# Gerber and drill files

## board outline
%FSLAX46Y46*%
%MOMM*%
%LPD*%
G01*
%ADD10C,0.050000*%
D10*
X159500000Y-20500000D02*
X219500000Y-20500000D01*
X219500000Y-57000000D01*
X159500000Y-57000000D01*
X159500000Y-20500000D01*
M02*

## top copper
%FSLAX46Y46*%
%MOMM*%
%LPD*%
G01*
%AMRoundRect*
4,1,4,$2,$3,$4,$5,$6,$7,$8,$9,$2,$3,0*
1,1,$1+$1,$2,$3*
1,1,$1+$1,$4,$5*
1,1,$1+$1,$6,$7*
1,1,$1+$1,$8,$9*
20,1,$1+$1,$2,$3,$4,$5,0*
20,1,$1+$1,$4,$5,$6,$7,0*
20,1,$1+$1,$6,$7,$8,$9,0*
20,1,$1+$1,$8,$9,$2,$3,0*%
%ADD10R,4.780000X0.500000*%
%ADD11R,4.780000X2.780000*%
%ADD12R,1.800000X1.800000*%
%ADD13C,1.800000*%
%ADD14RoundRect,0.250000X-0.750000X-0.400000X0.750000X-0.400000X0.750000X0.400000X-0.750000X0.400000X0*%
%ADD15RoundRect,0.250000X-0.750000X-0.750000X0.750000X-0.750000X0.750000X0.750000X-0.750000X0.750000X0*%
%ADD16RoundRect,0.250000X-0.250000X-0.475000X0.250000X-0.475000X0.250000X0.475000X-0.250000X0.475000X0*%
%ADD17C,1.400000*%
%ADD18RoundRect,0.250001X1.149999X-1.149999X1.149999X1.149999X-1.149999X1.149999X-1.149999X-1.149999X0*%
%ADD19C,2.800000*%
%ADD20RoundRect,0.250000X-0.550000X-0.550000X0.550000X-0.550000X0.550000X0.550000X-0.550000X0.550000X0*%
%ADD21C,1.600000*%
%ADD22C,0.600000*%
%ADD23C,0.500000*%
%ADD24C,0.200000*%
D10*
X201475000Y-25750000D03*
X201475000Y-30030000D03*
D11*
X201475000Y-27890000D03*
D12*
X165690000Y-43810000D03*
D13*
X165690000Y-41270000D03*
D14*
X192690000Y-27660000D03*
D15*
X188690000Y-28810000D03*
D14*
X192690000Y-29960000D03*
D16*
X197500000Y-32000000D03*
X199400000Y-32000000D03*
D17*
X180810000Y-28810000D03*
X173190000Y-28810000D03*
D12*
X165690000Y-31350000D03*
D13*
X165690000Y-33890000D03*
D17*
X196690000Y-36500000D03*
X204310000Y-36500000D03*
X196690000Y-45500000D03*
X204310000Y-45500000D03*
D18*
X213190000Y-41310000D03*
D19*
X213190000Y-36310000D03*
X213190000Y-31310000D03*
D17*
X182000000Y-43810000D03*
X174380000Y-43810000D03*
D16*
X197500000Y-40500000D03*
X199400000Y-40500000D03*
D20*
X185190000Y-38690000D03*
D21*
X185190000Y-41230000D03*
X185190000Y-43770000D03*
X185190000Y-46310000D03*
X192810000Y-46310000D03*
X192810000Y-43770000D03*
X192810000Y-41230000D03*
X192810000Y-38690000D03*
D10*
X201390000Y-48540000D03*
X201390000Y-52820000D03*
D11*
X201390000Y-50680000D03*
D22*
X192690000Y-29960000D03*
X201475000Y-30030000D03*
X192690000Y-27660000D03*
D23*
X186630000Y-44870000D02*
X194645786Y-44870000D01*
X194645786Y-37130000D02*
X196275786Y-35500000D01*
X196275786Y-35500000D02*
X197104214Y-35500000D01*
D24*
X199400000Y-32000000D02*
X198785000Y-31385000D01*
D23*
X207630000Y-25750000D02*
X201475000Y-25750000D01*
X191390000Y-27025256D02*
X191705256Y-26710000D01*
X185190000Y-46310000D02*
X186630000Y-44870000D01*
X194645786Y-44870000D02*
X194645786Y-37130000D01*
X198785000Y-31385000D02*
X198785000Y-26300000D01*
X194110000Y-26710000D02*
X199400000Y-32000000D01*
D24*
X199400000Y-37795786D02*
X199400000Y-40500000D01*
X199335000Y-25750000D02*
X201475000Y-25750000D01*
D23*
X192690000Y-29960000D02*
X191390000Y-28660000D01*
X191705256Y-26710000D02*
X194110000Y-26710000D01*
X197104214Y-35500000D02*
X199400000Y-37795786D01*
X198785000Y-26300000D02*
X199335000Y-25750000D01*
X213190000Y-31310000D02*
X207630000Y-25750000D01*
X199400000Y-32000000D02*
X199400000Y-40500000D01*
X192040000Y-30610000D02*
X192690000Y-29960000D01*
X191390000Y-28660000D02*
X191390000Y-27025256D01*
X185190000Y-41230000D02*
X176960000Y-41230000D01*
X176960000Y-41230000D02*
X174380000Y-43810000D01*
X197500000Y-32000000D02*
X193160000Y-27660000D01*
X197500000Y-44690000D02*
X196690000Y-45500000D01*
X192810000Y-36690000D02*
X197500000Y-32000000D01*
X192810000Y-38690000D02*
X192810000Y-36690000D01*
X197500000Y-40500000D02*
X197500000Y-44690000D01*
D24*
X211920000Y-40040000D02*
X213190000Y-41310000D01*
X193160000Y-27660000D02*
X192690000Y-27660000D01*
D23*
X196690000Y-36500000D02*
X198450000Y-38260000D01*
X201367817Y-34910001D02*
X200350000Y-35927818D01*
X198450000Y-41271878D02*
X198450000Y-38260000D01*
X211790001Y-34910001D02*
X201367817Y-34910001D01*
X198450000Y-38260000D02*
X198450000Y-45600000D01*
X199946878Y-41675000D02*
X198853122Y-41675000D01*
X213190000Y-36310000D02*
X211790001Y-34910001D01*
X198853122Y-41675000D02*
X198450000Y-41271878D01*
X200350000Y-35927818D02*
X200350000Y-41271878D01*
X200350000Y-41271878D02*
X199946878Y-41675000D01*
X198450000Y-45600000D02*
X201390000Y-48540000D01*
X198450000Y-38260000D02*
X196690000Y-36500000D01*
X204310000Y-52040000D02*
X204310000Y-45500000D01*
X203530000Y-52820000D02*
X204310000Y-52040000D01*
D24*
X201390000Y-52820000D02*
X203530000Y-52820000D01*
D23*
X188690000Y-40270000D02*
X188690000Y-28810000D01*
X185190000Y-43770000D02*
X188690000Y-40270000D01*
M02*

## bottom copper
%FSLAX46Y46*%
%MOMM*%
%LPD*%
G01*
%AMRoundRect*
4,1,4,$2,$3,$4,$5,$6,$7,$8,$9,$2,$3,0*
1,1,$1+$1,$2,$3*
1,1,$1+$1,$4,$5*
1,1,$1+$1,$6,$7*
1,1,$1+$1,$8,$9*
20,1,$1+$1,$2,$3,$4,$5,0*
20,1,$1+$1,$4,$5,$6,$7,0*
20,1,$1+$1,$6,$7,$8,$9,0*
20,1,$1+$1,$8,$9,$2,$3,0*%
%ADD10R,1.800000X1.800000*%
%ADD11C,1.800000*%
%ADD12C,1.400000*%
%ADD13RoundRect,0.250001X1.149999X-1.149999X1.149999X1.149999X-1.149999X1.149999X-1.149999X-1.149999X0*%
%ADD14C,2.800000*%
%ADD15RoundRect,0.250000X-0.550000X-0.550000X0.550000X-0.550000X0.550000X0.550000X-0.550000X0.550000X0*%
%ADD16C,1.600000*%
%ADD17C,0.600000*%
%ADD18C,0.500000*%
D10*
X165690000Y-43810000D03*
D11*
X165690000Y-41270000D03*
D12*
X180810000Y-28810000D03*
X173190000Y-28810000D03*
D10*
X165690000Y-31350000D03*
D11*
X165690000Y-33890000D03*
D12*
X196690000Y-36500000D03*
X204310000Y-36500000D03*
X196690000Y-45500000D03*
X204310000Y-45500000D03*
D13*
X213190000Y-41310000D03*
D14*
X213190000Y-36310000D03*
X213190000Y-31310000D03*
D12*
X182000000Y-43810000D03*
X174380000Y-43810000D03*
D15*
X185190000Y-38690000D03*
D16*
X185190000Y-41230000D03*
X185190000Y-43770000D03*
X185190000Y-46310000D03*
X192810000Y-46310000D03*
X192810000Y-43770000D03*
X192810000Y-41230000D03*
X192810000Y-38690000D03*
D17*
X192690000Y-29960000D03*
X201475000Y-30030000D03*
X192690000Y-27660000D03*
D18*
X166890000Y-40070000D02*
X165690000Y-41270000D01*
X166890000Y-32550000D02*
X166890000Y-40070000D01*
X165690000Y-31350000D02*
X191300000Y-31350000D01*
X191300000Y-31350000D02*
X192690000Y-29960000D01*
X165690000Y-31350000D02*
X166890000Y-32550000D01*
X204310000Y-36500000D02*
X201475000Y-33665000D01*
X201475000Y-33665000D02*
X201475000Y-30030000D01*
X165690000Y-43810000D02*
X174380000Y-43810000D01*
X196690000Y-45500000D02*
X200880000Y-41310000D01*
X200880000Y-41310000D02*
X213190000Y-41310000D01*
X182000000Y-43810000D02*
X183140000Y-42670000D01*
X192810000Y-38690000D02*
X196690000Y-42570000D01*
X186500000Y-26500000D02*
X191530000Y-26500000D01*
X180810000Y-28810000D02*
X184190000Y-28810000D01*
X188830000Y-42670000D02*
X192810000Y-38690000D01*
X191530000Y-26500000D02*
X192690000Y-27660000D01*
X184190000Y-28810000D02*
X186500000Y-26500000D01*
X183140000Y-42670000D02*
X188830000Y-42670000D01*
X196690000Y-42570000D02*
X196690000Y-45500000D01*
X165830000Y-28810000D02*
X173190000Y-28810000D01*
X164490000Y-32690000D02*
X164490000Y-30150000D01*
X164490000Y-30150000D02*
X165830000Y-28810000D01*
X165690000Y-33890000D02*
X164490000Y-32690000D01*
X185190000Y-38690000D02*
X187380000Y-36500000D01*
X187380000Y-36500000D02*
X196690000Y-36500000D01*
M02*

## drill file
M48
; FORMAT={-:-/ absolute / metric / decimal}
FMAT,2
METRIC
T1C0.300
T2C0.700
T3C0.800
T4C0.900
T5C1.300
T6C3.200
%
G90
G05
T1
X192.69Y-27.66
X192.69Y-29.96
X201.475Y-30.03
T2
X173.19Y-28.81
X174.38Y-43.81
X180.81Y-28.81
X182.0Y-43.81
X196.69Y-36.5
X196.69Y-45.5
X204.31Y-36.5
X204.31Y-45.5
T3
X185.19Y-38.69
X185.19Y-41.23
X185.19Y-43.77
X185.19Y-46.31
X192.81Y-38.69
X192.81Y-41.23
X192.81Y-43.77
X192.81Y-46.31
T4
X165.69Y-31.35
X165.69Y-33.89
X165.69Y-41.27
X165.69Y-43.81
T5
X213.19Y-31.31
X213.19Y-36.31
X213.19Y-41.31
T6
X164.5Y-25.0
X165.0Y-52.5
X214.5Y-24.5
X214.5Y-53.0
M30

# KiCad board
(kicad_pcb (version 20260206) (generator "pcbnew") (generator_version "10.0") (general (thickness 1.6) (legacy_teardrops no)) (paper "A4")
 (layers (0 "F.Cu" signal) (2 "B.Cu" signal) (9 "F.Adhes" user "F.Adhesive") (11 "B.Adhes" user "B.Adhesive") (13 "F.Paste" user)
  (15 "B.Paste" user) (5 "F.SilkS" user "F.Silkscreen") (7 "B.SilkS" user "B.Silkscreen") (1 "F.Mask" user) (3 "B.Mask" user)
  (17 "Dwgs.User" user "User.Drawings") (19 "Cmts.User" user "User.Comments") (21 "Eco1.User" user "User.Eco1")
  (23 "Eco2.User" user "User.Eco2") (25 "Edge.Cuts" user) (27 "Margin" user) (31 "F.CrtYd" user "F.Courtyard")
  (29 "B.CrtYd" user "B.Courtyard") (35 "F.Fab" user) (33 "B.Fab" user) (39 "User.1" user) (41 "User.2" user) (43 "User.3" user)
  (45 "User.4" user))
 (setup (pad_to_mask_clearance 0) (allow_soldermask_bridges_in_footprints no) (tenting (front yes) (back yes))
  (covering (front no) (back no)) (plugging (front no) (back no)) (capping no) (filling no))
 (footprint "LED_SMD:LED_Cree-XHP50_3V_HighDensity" (layer "F.Cu") (at 201.475 27.89 -90)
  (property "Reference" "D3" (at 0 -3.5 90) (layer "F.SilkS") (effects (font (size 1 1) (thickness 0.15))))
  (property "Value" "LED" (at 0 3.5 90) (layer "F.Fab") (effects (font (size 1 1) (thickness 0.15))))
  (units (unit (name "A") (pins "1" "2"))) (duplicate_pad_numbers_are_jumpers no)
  (pad "" smd rect (at -2.14 -1.32 270) (size 0.5 2.14) (layers "F.Paste"))
  (pad "" smd rect (at -2.14 1.32 270) (size 0.5 2.14) (layers "F.Paste"))
  (pad "" smd rect (at -0.61 -1.575 270) (size 0.97 0.8) (layers "F.Paste"))
  (pad "" smd rect (at -0.61 -0.525 270) (size 0.97 0.8) (layers "F.Paste"))
  (pad "" smd rect (at -0.61 0.525 270) (size 0.97 0.8) (layers "F.Paste"))
  (pad "" smd rect (at -0.61 1.575 270) (size 0.97 0.8) (layers "F.Paste"))
  (pad "" smd rect (at 0.61 -1.575 270) (size 0.97 0.8) (layers "F.Paste"))
  (pad "" smd rect (at 0.61 -0.525 270) (size 0.97 0.8) (layers "F.Paste"))
  (pad "" smd rect (at 0.61 0.525 270) (size 0.97 0.8) (layers "F.Paste"))
  (pad "" smd rect (at 0.61 1.575 270) (size 0.97 0.8) (layers "F.Paste"))
  (pad "" smd rect (at 2.14 -1.32 270) (size 0.5 2.14) (layers "F.Paste"))
  (pad "" smd rect (at 2.14 1.32 270) (size 0.5 2.14) (layers "F.Paste"))
  (pad "1" smd rect (at -2.14 0 270) (size 0.5 4.78) (layers "F.Cu" "F.Mask") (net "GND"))
  (pad "2" smd rect (at 2.14 0 270) (size 0.5 4.78) (layers "F.Cu" "F.Mask") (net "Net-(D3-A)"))
  (pad "3" smd rect (at 0 0 270) (size 2.78 4.78) (layers "F.Cu" "F.Mask")))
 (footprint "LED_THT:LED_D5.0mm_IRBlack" (layer "F.Cu") (at 165.69 43.81 90)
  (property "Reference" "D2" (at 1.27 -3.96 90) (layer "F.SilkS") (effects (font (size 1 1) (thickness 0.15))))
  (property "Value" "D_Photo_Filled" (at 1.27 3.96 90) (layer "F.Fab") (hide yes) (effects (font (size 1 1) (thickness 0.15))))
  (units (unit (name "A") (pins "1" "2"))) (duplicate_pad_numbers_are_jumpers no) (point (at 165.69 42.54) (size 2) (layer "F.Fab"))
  (pad "1" thru_hole rect (at 0 0 90) (size 1.8 1.8) (drill 0.9) (layers "*.Cu" "*.Mask") (remove_unused_layers no) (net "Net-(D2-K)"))
  (pad "2" thru_hole circle (at 2.54 0 90) (size 1.8 1.8) (drill 0.9) (layers "*.Cu" "*.Mask") (remove_unused_layers no) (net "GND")))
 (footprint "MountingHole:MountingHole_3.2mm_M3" (layer "F.Cu") (at 165 52.5)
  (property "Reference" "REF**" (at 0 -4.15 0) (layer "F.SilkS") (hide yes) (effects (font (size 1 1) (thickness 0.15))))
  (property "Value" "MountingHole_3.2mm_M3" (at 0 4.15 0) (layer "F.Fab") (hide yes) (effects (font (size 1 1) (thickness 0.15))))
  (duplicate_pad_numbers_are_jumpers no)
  (pad "" np_thru_hole circle (at 0 0) (size 3.2 3.2) (drill 3.2) (layers "*.Cu" "*.Mask")))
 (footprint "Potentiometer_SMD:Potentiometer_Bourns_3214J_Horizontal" (layer "F.Cu") (at 190.69 28.81)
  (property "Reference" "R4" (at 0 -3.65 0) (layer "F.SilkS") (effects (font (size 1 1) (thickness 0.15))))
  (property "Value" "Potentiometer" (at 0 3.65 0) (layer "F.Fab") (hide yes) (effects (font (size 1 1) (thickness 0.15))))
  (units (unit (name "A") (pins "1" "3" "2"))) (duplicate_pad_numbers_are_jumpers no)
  (pad "1" smd roundrect (at 2 -1.15) (size 2 1.3) (layers "F.Cu" "F.Mask" "F.Paste") (roundrect_rratio 0.192308) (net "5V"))
  (pad "2" smd roundrect (at -2 0) (size 2 2) (layers "F.Cu" "F.Mask" "F.Paste") (roundrect_rratio 0.125) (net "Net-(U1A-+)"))
  (pad "3" smd roundrect (at 2 1.15) (size 2 1.3) (layers "F.Cu" "F.Mask" "F.Paste") (roundrect_rratio 0.192308) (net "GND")))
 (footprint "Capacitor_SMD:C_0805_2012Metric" (layer "F.Cu") (at 198.45 32)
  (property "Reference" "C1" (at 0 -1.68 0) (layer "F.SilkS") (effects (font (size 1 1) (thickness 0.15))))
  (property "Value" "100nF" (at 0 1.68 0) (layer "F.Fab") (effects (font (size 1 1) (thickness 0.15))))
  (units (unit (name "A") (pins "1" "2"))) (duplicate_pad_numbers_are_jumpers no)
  (pad "1" smd roundrect (at -0.95 0) (size 1 1.45) (layers "F.Cu" "F.Mask" "F.Paste") (roundrect_rratio 0.25) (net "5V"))
  (pad "2" smd roundrect (at 0.95 0) (size 1 1.45) (layers "F.Cu" "F.Mask" "F.Paste") (roundrect_rratio 0.25) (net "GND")))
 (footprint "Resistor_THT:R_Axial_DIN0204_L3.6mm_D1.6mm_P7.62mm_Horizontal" (layer "F.Cu") (at 180.81 28.81 180)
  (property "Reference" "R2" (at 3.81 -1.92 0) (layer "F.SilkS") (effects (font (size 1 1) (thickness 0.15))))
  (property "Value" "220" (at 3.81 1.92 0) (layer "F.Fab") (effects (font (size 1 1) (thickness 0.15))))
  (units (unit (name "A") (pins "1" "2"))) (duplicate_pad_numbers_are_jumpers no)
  (pad "1" thru_hole circle (at 0 0 180) (size 1.4 1.4) (drill 0.7) (layers "*.Cu" "*.Mask") (remove_unused_layers no) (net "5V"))
  (pad "2" thru_hole circle (at 7.62 0 180) (size 1.4 1.4) (drill 0.7) (layers "*.Cu" "*.Mask") (remove_unused_layers no) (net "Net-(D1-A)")))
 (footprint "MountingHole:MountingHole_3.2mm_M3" (layer "F.Cu") (at 214.5 24.5)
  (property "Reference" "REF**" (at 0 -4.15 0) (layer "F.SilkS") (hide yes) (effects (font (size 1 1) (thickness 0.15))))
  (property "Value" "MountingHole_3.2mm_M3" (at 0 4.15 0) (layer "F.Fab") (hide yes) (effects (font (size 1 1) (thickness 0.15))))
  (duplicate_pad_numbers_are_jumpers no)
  (pad "" np_thru_hole circle (at 0 0) (size 3.2 3.2) (drill 3.2) (layers "*.Cu" "*.Mask")))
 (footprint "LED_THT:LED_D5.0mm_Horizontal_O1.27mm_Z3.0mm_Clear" (layer "F.Cu") (at 165.69 31.35 -90)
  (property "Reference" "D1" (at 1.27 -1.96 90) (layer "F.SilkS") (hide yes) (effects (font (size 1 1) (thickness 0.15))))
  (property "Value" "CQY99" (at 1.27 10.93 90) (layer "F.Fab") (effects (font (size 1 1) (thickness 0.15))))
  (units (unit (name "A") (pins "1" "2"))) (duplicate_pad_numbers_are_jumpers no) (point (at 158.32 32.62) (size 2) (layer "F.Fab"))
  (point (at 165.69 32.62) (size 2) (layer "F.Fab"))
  (pad "1" thru_hole rect (at 0 0 270) (size 1.8 1.8) (drill 0.9) (layers "*.Cu" "*.Mask") (remove_unused_layers no) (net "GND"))
  (pad "2" thru_hole circle (at 2.54 0 270) (size 1.8 1.8) (drill 0.9) (layers "*.Cu" "*.Mask") (remove_unused_layers no) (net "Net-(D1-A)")))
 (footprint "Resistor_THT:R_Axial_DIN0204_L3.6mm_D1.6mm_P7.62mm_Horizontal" (layer "F.Cu") (at 196.69 36.5)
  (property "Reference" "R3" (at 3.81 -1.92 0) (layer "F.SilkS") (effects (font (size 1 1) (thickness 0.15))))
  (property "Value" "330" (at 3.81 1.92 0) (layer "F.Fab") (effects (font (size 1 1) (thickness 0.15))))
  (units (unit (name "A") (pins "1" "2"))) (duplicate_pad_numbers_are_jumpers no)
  (pad "1" thru_hole circle (at 0 0) (size 1.4 1.4) (drill 0.7) (layers "*.Cu" "*.Mask") (remove_unused_layers no) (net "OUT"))
  (pad "2" thru_hole circle (at 7.62 0) (size 1.4 1.4) (drill 0.7) (layers "*.Cu" "*.Mask") (remove_unused_layers no) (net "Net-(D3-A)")))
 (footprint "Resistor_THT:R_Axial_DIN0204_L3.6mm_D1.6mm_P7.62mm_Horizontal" (layer "F.Cu") (at 196.69 45.5)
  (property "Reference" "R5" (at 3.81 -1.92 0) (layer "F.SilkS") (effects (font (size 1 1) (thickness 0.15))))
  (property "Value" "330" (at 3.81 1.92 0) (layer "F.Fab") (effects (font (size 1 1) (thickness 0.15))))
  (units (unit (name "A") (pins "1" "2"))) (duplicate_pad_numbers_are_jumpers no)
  (pad "1" thru_hole circle (at 0 0) (size 1.4 1.4) (drill 0.7) (layers "*.Cu" "*.Mask") (remove_unused_layers no) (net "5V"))
  (pad "2" thru_hole circle (at 7.62 0) (size 1.4 1.4) (drill 0.7) (layers "*.Cu" "*.Mask") (remove_unused_layers no) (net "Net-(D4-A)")))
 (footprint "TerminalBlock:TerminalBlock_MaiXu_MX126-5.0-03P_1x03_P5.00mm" (layer "F.Cu") (at 213.19 41.31 90)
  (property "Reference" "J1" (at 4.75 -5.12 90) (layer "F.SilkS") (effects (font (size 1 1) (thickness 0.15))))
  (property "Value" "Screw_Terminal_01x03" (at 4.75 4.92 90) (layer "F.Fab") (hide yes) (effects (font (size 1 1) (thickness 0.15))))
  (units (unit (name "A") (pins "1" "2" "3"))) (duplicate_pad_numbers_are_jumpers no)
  (pad "1" thru_hole roundrect (at 0 0 90) (size 2.8 2.8) (drill 1.3) (layers "*.Cu" "*.Mask") (remove_unused_layers no)
   (roundrect_rratio 0.089286) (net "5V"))
  (pad "2" thru_hole circle (at 5 0 90) (size 2.8 2.8) (drill 1.3) (layers "*.Cu" "*.Mask") (remove_unused_layers no) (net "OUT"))
  (pad "3" thru_hole circle (at 10 0 90) (size 2.8 2.8) (drill 1.3) (layers "*.Cu" "*.Mask") (remove_unused_layers no) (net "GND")))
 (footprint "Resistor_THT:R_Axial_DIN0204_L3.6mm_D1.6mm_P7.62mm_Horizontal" (layer "F.Cu") (at 182 43.81 180)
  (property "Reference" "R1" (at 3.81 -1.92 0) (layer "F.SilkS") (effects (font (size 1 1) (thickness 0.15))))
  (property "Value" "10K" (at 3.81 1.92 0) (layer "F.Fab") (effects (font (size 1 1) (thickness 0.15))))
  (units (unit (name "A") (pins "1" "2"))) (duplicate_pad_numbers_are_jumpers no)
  (pad "1" thru_hole circle (at 0 0 180) (size 1.4 1.4) (drill 0.7) (layers "*.Cu" "*.Mask") (remove_unused_layers no) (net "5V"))
  (pad "2" thru_hole circle (at 7.62 0 180) (size 1.4 1.4) (drill 0.7) (layers "*.Cu" "*.Mask") (remove_unused_layers no) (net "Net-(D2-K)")))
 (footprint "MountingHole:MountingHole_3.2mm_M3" (layer "F.Cu") (at 214.5 53)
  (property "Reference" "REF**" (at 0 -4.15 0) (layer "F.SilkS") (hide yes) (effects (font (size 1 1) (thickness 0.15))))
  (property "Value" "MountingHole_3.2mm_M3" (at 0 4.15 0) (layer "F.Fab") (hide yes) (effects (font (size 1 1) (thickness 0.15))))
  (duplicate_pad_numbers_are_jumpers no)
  (pad "" np_thru_hole circle (at 0 0) (size 3.2 3.2) (drill 3.2) (layers "*.Cu" "*.Mask")))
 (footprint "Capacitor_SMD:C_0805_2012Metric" (layer "F.Cu") (at 198.45 40.5)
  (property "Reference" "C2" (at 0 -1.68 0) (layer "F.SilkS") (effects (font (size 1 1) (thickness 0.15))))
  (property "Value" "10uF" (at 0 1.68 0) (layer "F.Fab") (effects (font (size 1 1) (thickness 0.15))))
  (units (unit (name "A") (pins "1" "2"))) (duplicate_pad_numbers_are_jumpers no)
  (pad "1" smd roundrect (at -0.95 0) (size 1 1.45) (layers "F.Cu" "F.Mask" "F.Paste") (roundrect_rratio 0.25) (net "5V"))
  (pad "2" smd roundrect (at 0.95 0) (size 1 1.45) (layers "F.Cu" "F.Mask" "F.Paste") (roundrect_rratio 0.25) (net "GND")))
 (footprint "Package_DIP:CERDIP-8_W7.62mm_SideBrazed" (layer "F.Cu") (at 185.19 38.69)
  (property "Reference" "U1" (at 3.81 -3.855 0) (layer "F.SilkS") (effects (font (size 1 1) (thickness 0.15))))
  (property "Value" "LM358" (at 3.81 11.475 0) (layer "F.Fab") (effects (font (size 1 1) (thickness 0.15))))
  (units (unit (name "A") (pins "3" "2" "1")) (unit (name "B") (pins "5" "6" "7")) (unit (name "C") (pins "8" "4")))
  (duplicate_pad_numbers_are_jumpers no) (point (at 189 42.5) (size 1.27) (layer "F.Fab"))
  (pad "1" thru_hole roundrect (at 0 0) (size 1.6 1.6) (drill 0.8) (layers "*.Cu" "*.Mask") (remove_unused_layers no)
   (roundrect_rratio 0.15625) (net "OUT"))
  (pad "2" thru_hole circle (at 0 2.54) (size 1.6 1.6) (drill 0.8) (layers "*.Cu" "*.Mask") (remove_unused_layers no) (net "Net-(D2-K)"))
  (pad "3" thru_hole circle (at 0 5.08) (size 1.6 1.6) (drill 0.8) (layers "*.Cu" "*.Mask") (remove_unused_layers no) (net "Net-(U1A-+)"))
  (pad "4" thru_hole circle (at 0 7.62) (size 1.6 1.6) (drill 0.8) (layers "*.Cu" "*.Mask") (remove_unused_layers no) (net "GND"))
  (pad "5" thru_hole circle (at 7.62 7.62) (size 1.6 1.6) (drill 0.8) (layers "*.Cu" "*.Mask") (remove_unused_layers no))
  (pad "6" thru_hole circle (at 7.62 5.08) (size 1.6 1.6) (drill 0.8) (layers "*.Cu" "*.Mask") (remove_unused_layers no))
  (pad "7" thru_hole circle (at 7.62 2.54) (size 1.6 1.6) (drill 0.8) (layers "*.Cu" "*.Mask") (remove_unused_layers no))
  (pad "8" thru_hole circle (at 7.62 0) (size 1.6 1.6) (drill 0.8) (layers "*.Cu" "*.Mask") (remove_unused_layers no) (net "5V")))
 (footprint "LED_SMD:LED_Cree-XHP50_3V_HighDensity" (layer "F.Cu") (at 201.39 50.68 -90)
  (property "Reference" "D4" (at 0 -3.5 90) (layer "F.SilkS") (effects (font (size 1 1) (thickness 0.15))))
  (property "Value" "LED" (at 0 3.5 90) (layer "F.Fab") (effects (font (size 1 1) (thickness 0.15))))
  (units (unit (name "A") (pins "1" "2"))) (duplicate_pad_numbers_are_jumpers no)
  (pad "" smd rect (at -2.14 -1.32 270) (size 0.5 2.14) (layers "F.Paste"))
  (pad "" smd rect (at -2.14 1.32 270) (size 0.5 2.14) (layers "F.Paste"))
  (pad "" smd rect (at -0.61 -1.575 270) (size 0.97 0.8) (layers "F.Paste"))
  (pad "" smd rect (at -0.61 -0.525 270) (size 0.97 0.8) (layers "F.Paste"))
  (pad "" smd rect (at -0.61 0.525 270) (size 0.97 0.8) (layers "F.Paste"))
  (pad "" smd rect (at -0.61 1.575 270) (size 0.97 0.8) (layers "F.Paste"))
  (pad "" smd rect (at 0.61 -1.575 270) (size 0.97 0.8) (layers "F.Paste"))
  (pad "" smd rect (at 0.61 -0.525 270) (size 0.97 0.8) (layers "F.Paste"))
  (pad "" smd rect (at 0.61 0.525 270) (size 0.97 0.8) (layers "F.Paste"))
  (pad "" smd rect (at 0.61 1.575 270) (size 0.97 0.8) (layers "F.Paste"))
  (pad "" smd rect (at 2.14 -1.32 270) (size 0.5 2.14) (layers "F.Paste"))
  (pad "" smd rect (at 2.14 1.32 270) (size 0.5 2.14) (layers "F.Paste"))
  (pad "1" smd rect (at -2.14 0 270) (size 0.5 4.78) (layers "F.Cu" "F.Mask") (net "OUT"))
  (pad "2" smd rect (at 2.14 0 270) (size 0.5 4.78) (layers "F.Cu" "F.Mask") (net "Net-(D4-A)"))
  (pad "3" smd rect (at 0 0 270) (size 2.78 4.78) (layers "F.Cu" "F.Mask")))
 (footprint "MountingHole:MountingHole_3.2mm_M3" (layer "F.Cu") (at 164.5 25)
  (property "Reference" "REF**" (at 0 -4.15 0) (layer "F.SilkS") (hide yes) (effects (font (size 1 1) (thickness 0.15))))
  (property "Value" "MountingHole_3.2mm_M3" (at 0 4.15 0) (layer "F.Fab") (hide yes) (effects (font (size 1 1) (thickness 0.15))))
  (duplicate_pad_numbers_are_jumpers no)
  (pad "" np_thru_hole circle (at 0 0) (size 3.2 3.2) (drill 3.2) (layers "*.Cu" "*.Mask")))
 (gr_rect (start 159.5 20.5) (end 219.5 57) (stroke (width 0.05) (type default)) (fill no) (layer "Edge.Cuts"))
 (segment (start 186.63 44.87) (end 194.645786 44.87) (width 0.5) (layer "F.Cu") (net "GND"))
 (segment (start 194.645786 37.13) (end 196.275786 35.5) (width 0.5) (layer "F.Cu") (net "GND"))
 (segment (start 196.275786 35.5) (end 197.104214 35.5) (width 0.5) (layer "F.Cu") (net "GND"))
 (segment (start 199.4 32) (end 198.785 31.385) (width 0.2) (layer "F.Cu") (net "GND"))
 (segment (start 207.63 25.75) (end 201.475 25.75) (width 0.5) (layer "F.Cu") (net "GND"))
 (segment (start 191.39 27.025256) (end 191.705256 26.71) (width 0.5) (layer "F.Cu") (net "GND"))
 (segment (start 185.19 46.31) (end 186.63 44.87) (width 0.5) (layer "F.Cu") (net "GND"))
 (segment (start 194.645786 44.87) (end 194.645786 37.13) (width 0.5) (layer "F.Cu") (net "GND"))
 (segment (start 198.785 31.385) (end 198.785 26.3) (width 0.5) (layer "F.Cu") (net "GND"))
 (segment (start 194.11 26.71) (end 199.4 32) (width 0.5) (layer "F.Cu") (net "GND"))
 (segment (start 199.4 37.795786) (end 199.4 40.5) (width 0.2) (layer "F.Cu") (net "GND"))
 (segment (start 199.335 25.75) (end 201.475 25.75) (width 0.2) (layer "F.Cu") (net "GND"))
 (segment (start 192.69 29.96) (end 191.39 28.66) (width 0.5) (layer "F.Cu") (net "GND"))
 (segment (start 191.705256 26.71) (end 194.11 26.71) (width 0.5) (layer "F.Cu") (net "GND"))
 (segment (start 197.104214 35.5) (end 199.4 37.795786) (width 0.5) (layer "F.Cu") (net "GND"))
 (segment (start 198.785 26.3) (end 199.335 25.75) (width 0.5) (layer "F.Cu") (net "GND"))
 (segment (start 213.19 31.31) (end 207.63 25.75) (width 0.5) (layer "F.Cu") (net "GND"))
 (segment (start 199.4 32) (end 199.4 40.5) (width 0.5) (layer "F.Cu") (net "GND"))
 (segment (start 192.04 30.61) (end 192.69 29.96) (width 0.5) (layer "F.Cu") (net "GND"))
 (segment (start 191.39 28.66) (end 191.39 27.025256) (width 0.5) (layer "F.Cu") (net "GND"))
 (via (at 192.69 29.96) (size 0.6) (drill 0.3) (layers "F.Cu" "B.Cu") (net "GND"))
 (segment (start 166.89 40.07) (end 165.69 41.27) (width 0.5) (layer "B.Cu") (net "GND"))
 (segment (start 166.89 32.55) (end 166.89 40.07) (width 0.5) (layer "B.Cu") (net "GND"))
 (segment (start 165.69 31.35) (end 191.3 31.35) (width 0.5) (layer "B.Cu") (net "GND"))
 (segment (start 191.3 31.35) (end 192.69 29.96) (width 0.5) (layer "B.Cu") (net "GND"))
 (segment (start 165.69 31.35) (end 166.89 32.55) (width 0.5) (layer "B.Cu") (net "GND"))
 (via (at 201.475 30.03) (size 0.6) (drill 0.3) (layers "F.Cu" "B.Cu") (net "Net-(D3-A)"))
 (segment (start 204.31 36.5) (end 201.475 33.665) (width 0.5) (layer "B.Cu") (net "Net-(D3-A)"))
 (segment (start 201.475 33.665) (end 201.475 30.03) (width 0.5) (layer "B.Cu") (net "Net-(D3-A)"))
 (segment (start 185.19 41.23) (end 176.96 41.23) (width 0.5) (layer "F.Cu") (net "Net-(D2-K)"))
 (segment (start 176.96 41.23) (end 174.38 43.81) (width 0.5) (layer "F.Cu") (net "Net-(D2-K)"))
 (segment (start 165.69 43.81) (end 174.38 43.81) (width 0.5) (layer "B.Cu") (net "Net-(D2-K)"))
 (segment (start 197.5 32) (end 193.16 27.66) (width 0.5) (layer "F.Cu") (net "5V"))
 (segment (start 197.5 44.69) (end 196.69 45.5) (width 0.5) (layer "F.Cu") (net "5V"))
 (segment (start 192.81 36.69) (end 197.5 32) (width 0.5) (layer "F.Cu") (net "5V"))
 (segment (start 192.81 38.69) (end 192.81 36.69) (width 0.5) (layer "F.Cu") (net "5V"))
 (segment (start 197.5 40.5) (end 197.5 44.69) (width 0.5) (layer "F.Cu") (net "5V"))
 (segment (start 211.92 40.04) (end 213.19 41.31) (width 0.2) (layer "F.Cu") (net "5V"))
 (segment (start 193.16 27.66) (end 192.69 27.66) (width 0.2) (layer "F.Cu") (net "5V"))
 (via (at 192.69 27.66) (size 0.6) (drill 0.3) (layers "F.Cu" "B.Cu") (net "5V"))
 (segment (start 196.69 45.5) (end 200.88 41.31) (width 0.5) (layer "B.Cu") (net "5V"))
 (segment (start 200.88 41.31) (end 213.19 41.31) (width 0.5) (layer "B.Cu") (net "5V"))
 (segment (start 182 43.81) (end 183.14 42.67) (width 0.5) (layer "B.Cu") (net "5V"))
 (segment (start 192.81 38.69) (end 196.69 42.57) (width 0.5) (layer "B.Cu") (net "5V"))
 (segment (start 186.5 26.5) (end 191.53 26.5) (width 0.5) (layer "B.Cu") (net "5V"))
 (segment (start 180.81 28.81) (end 184.19 28.81) (width 0.5) (layer "B.Cu") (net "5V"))
 (segment (start 188.83 42.67) (end 192.81 38.69) (width 0.5) (layer "B.Cu") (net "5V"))
 (segment (start 191.53 26.5) (end 192.69 27.66) (width 0.5) (layer "B.Cu") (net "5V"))
 (segment (start 184.19 28.81) (end 186.5 26.5) (width 0.5) (layer "B.Cu") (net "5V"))
 (segment (start 183.14 42.67) (end 188.83 42.67) (width 0.5) (layer "B.Cu") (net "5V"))
 (segment (start 196.69 42.57) (end 196.69 45.5) (width 0.5) (layer "B.Cu") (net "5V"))
 (segment (start 165.83 28.81) (end 173.19 28.81) (width 0.5) (layer "B.Cu") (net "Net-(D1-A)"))
 (segment (start 164.49 32.69) (end 164.49 30.15) (width 0.5) (layer "B.Cu") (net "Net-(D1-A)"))
 (segment (start 164.49 30.15) (end 165.83 28.81) (width 0.5) (layer "B.Cu") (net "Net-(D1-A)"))
 (segment (start 165.69 33.89) (end 164.49 32.69) (width 0.5) (layer "B.Cu") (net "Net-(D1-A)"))
 (segment (start 196.69 36.5) (end 198.45 38.26) (width 0.5) (layer "F.Cu") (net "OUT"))
 (segment (start 201.367817 34.910001) (end 200.35 35.927818) (width 0.5) (layer "F.Cu") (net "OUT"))
 (segment (start 198.45 41.271878) (end 198.45 38.26) (width 0.5) (layer "F.Cu") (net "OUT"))
 (segment (start 211.790001 34.910001) (end 201.367817 34.910001) (width 0.5) (layer "F.Cu") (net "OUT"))
 (segment (start 198.45 38.26) (end 198.45 45.6) (width 0.5) (layer "F.Cu") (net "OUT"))
 (segment (start 199.946878 41.675) (end 198.853122 41.675) (width 0.5) (layer "F.Cu") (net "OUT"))
 (segment (start 213.19 36.31) (end 211.790001 34.910001) (width 0.5) (layer "F.Cu") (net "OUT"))
 (segment (start 198.853122 41.675) (end 198.45 41.271878) (width 0.5) (layer "F.Cu") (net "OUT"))
 (segment (start 200.35 35.927818) (end 200.35 41.271878) (width 0.5) (layer "F.Cu") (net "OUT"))
 (segment (start 200.35 41.271878) (end 199.946878 41.675) (width 0.5) (layer "F.Cu") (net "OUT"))
 (segment (start 198.45 45.6) (end 201.39 48.54) (width 0.5) (layer "F.Cu") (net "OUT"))
 (segment (start 198.45 38.26) (end 196.69 36.5) (width 0.5) (layer "F.Cu") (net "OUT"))
 (segment (start 185.19 38.69) (end 187.38 36.5) (width 0.5) (layer "B.Cu") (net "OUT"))
 (segment (start 187.38 36.5) (end 196.69 36.5) (width 0.5) (layer "B.Cu") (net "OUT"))
 (segment (start 204.31 52.04) (end 204.31 45.5) (width 0.5) (layer "F.Cu") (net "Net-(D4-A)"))
 (segment (start 203.53 52.82) (end 204.31 52.04) (width 0.5) (layer "F.Cu") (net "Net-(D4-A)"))
 (segment (start 201.39 52.82) (end 203.53 52.82) (width 0.2) (layer "F.Cu") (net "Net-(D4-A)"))
 (segment (start 188.69 40.27) (end 188.69 28.81) (width 0.5) (layer "F.Cu") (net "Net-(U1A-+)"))
 (segment (start 185.19 43.77) (end 188.69 40.27) (width 0.5) (layer "F.Cu") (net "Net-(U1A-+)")))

